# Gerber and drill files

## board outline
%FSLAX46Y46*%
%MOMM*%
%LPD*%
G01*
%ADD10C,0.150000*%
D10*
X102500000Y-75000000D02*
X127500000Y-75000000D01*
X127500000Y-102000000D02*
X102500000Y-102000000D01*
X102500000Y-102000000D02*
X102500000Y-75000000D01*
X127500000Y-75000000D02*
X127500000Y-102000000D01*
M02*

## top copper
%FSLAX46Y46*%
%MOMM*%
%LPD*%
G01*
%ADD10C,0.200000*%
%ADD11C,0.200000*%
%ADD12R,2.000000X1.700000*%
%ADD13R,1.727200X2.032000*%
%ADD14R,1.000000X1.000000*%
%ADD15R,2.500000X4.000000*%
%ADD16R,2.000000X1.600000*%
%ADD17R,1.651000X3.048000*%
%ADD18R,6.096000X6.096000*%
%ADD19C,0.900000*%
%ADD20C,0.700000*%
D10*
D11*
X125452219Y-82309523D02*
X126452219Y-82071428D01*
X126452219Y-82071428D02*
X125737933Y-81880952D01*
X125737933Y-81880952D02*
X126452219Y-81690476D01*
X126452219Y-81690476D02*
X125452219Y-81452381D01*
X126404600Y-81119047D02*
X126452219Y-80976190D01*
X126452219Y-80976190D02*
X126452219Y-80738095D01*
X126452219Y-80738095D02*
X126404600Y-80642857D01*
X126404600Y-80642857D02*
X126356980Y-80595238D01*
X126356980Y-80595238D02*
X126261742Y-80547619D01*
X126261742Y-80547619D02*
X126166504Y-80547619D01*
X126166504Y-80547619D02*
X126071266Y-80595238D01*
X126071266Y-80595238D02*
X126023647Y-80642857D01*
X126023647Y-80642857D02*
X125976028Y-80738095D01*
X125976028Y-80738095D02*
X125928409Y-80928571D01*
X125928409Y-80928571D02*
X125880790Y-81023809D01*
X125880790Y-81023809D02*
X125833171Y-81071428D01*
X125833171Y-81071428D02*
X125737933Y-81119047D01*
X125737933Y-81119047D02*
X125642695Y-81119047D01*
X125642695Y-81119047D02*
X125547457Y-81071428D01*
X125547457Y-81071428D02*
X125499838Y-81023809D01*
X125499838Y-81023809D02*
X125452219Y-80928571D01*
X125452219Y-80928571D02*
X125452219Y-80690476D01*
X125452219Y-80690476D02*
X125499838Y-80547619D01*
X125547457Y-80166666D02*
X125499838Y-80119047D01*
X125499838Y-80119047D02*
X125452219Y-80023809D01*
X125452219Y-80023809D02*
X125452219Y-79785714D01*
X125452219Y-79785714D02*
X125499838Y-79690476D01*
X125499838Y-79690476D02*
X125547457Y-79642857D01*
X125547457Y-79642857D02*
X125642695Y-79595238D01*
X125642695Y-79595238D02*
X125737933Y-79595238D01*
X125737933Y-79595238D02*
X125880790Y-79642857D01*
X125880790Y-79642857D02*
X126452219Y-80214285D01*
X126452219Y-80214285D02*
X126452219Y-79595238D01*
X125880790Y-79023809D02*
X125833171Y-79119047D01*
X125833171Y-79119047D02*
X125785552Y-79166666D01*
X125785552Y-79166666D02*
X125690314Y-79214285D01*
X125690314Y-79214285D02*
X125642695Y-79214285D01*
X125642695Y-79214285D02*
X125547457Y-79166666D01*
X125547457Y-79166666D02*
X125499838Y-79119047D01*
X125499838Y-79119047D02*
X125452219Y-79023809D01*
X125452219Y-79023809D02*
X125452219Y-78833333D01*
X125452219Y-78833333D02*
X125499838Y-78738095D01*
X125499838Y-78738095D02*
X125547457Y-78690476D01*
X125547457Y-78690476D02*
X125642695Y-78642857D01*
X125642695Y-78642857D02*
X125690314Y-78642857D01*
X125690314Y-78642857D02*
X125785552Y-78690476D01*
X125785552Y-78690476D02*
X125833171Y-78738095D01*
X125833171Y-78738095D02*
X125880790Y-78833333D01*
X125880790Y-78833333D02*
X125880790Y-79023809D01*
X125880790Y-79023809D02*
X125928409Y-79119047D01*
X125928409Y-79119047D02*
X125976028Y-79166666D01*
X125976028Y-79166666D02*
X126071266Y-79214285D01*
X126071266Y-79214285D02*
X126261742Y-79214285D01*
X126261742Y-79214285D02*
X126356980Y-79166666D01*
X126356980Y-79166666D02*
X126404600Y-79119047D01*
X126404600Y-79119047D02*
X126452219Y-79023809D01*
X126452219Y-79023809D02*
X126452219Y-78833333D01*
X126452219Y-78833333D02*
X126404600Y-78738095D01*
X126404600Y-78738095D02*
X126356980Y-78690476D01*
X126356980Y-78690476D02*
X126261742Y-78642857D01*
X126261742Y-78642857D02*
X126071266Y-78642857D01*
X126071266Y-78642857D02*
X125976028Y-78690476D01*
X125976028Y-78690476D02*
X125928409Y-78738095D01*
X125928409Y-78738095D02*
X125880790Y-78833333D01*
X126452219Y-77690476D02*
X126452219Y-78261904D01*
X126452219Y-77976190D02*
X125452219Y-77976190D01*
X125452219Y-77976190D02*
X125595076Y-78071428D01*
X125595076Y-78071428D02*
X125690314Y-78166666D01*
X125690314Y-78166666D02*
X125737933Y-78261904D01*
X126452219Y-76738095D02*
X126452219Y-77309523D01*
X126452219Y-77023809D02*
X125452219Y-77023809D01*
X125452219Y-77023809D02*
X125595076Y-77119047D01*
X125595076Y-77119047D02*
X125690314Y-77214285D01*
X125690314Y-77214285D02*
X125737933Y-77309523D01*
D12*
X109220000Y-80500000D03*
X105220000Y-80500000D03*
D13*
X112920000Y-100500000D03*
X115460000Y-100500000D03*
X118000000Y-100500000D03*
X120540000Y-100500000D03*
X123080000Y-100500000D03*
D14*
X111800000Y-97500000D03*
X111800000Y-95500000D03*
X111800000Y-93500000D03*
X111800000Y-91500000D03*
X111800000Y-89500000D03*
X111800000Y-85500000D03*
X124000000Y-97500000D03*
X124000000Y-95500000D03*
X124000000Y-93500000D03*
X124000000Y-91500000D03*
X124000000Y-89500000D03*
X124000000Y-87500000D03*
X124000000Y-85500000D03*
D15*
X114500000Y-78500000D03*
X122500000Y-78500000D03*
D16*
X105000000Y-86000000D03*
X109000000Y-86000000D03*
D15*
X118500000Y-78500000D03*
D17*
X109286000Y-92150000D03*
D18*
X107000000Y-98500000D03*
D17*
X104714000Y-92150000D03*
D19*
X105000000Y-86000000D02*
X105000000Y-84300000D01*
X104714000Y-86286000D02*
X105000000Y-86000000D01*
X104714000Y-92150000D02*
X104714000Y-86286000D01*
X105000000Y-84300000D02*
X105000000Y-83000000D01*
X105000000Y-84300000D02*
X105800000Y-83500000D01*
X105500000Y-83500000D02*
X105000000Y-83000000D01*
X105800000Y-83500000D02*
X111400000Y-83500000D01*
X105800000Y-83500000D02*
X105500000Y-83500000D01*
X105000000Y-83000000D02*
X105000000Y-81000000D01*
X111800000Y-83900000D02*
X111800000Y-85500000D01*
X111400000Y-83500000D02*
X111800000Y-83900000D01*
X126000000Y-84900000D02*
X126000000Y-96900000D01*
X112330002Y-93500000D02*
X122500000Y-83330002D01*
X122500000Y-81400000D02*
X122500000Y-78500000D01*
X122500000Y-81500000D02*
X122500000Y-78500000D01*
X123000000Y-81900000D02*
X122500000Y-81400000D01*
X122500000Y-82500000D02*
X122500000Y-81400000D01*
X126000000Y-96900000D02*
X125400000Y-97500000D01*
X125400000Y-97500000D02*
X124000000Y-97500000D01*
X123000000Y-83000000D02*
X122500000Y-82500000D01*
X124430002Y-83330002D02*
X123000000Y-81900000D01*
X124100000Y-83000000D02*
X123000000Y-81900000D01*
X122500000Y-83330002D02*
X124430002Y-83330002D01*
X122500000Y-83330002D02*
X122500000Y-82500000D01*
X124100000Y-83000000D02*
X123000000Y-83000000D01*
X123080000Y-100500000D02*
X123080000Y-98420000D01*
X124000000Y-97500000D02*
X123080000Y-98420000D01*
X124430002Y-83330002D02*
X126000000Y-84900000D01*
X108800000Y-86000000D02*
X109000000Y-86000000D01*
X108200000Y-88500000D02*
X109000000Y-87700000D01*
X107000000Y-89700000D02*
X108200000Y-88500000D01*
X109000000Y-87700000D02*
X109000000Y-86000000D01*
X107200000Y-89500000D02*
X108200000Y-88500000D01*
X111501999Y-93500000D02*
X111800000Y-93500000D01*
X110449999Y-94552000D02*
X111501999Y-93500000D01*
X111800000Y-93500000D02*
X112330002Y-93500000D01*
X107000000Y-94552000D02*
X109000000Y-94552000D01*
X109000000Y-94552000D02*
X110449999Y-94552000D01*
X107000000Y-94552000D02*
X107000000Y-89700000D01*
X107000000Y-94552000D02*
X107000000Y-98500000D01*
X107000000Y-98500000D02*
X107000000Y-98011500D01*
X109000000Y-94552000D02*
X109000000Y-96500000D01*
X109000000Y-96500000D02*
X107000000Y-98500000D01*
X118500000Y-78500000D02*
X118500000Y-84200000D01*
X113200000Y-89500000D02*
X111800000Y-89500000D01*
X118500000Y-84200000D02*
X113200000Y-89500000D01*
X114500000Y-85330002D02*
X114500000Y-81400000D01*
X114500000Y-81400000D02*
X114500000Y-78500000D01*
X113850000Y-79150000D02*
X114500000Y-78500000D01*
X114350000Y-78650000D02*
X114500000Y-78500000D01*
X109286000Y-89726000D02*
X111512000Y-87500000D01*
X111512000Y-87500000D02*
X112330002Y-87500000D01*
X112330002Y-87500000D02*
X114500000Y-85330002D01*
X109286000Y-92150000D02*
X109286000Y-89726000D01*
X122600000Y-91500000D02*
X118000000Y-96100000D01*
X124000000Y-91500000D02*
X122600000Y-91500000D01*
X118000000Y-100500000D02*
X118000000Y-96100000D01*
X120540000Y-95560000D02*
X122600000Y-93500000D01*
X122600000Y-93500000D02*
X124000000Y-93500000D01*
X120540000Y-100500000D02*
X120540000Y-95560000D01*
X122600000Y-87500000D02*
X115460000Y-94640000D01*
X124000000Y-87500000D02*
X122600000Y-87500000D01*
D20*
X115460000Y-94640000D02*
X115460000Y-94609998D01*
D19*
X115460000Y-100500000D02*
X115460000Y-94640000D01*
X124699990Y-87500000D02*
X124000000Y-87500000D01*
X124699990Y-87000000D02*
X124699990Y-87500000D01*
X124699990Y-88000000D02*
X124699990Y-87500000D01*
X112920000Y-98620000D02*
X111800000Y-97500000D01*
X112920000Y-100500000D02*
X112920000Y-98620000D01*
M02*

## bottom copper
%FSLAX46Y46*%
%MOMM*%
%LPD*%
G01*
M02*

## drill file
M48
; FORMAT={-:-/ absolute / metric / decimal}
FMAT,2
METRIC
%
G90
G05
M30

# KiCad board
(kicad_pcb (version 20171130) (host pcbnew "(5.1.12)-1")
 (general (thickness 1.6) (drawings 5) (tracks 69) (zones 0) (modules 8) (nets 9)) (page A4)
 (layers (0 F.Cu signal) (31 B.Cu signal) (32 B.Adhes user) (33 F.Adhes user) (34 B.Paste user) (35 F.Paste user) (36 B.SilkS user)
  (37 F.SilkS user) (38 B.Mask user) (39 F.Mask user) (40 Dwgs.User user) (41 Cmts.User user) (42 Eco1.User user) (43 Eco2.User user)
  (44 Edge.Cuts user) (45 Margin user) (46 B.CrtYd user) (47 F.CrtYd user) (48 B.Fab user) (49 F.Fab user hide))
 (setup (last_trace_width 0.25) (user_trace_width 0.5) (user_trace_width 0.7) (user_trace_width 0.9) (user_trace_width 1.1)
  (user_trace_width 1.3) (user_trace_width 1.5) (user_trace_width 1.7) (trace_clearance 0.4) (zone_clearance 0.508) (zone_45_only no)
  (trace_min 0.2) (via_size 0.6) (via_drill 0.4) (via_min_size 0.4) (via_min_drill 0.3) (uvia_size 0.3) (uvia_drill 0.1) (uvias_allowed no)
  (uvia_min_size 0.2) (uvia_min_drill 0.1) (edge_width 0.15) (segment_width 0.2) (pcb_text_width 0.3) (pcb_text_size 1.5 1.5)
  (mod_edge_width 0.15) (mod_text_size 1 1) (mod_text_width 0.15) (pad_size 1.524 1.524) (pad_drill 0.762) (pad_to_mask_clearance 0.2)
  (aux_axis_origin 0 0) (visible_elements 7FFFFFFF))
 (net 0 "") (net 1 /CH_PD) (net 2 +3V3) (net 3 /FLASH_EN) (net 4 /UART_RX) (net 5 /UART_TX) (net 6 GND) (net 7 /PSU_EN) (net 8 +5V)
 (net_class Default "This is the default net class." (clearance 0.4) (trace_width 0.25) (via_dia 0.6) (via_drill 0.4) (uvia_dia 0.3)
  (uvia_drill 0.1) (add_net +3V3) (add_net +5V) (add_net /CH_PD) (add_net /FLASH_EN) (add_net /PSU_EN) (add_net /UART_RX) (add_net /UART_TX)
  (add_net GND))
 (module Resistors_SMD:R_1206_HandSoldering (layer F.Cu) (at 107.22 80.5 180)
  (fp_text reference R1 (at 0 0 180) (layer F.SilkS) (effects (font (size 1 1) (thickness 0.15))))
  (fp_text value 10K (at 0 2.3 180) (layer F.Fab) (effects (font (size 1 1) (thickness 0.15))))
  (pad 1 smd rect (at -2 0 180) (size 2 1.7) (layers F.Cu F.Paste F.Mask) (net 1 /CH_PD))
  (pad 2 smd rect (at 2 0 180) (size 2 1.7) (layers F.Cu F.Paste F.Mask) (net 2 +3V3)))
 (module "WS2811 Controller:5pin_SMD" (layer F.Cu) (at 112.92 100.5)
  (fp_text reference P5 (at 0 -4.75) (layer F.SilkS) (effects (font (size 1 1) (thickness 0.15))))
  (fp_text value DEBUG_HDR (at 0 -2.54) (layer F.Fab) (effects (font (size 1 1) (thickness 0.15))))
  (pad 1 smd rect (at 0 0) (size 1.7272 2.032) (layers F.Cu F.Paste F.Mask) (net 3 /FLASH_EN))
  (pad 2 smd rect (at 2.54 0) (size 1.7272 2.032) (layers F.Cu F.Paste F.Mask) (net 1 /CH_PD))
  (pad 3 smd rect (at 5.08 0) (size 1.7272 2.032) (layers F.Cu F.Paste F.Mask) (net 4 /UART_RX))
  (pad 4 smd rect (at 7.62 0) (size 1.7272 2.032) (layers F.Cu F.Paste F.Mask) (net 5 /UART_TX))
  (pad 5 smd rect (at 10.16 0) (size 1.7272 2.032) (layers F.Cu F.Paste F.Mask) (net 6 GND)))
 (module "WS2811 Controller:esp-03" (layer F.Cu) (at 117.9 91.6)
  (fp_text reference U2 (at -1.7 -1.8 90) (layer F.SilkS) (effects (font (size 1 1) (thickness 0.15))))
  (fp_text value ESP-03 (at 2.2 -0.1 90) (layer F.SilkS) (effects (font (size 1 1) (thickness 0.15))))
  (pad 14 smd rect (at -6.1 5.9) (size 1 1) (layers F.Cu F.Paste F.Mask) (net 3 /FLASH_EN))
  (pad 13 smd rect (at -6.1 3.9) (size 1 1) (layers F.Cu F.Paste F.Mask))
  (pad 12 smd rect (at -6.1 1.9) (size 1 1) (layers F.Cu F.Paste F.Mask) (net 6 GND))
  (pad 11 smd rect (at -6.1 -0.1) (size 1 1) (layers F.Cu F.Paste F.Mask))
  (pad 10 smd rect (at -6.1 -2.1) (size 1 1) (layers F.Cu F.Paste F.Mask) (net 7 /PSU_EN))
  (pad 8 smd rect (at -6.1 -6.1) (size 1 1) (layers F.Cu F.Paste F.Mask) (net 2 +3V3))
  (pad 1 smd rect (at 6.1 5.9) (size 1 1) (layers F.Cu F.Paste F.Mask) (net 6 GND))
  (pad 2 smd rect (at 6.1 3.9) (size 1 1) (layers F.Cu F.Paste F.Mask))
  (pad 3 smd rect (at 6.1 1.9) (size 1 1) (layers F.Cu F.Paste F.Mask) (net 5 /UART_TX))
  (pad 4 smd rect (at 6.1 -0.1) (size 1 1) (layers F.Cu F.Paste F.Mask) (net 4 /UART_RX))
  (pad 5 smd rect (at 6.1 -2.1) (size 1 1) (layers F.Cu F.Paste F.Mask))
  (pad 6 smd rect (at 6.1 -4.1) (size 1 1) (layers F.Cu F.Paste F.Mask) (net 1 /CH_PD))
  (pad 7 smd rect (at 6.1 -6.1) (size 1 1) (layers F.Cu F.Paste F.Mask)))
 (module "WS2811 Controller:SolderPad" (layer F.Cu) (at 114.5 78.5 270)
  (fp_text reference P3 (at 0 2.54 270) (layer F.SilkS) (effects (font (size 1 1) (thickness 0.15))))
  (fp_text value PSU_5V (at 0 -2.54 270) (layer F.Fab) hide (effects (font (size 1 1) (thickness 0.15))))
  (pad 1 smd rect (at 0 0 270) (size 4 2.5) (layers F.Cu F.Paste F.Mask) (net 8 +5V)))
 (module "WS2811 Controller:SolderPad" (layer F.Cu) (at 122.5 78.5 270)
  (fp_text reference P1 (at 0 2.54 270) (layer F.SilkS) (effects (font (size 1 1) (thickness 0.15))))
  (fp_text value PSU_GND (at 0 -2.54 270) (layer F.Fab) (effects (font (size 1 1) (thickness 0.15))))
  (pad 1 smd rect (at 0 0 270) (size 4 2.5) (layers F.Cu F.Paste F.Mask) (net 6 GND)))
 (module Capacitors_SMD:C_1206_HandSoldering (layer F.Cu) (at 107 86)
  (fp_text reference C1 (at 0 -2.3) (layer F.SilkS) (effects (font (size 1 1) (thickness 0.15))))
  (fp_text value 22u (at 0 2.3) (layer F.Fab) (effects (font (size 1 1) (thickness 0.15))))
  (pad 1 smd rect (at -2 0) (size 2 1.6) (layers F.Cu F.Paste F.Mask) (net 2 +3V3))
  (pad 2 smd rect (at 2 0) (size 2 1.6) (layers F.Cu F.Paste F.Mask) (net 6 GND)))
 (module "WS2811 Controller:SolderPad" (layer F.Cu) (at 118.5 78.5 90)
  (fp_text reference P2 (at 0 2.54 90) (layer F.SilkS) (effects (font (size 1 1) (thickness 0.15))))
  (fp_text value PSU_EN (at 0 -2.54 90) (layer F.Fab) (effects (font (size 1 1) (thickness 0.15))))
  (pad 1 smd rect (at 0 0 90) (size 4 2.5) (layers F.Cu F.Paste F.Mask) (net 7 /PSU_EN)))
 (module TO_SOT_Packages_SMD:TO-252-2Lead (layer F.Cu) (at 107 92.15 180)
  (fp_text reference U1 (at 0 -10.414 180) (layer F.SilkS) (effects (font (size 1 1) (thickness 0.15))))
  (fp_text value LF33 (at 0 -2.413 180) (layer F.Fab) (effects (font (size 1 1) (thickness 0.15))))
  (pad 1 smd rect (at -2.286 0 180) (size 1.651 3.048) (layers F.Cu F.Paste F.Mask) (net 8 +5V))
  (pad 2 smd rect (at 0 -6.35 180) (size 6.096 6.096) (layers F.Cu F.Paste F.Mask) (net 6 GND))
  (pad 3 smd rect (at 2.286 0 180) (size 1.651 3.048) (layers F.Cu F.Paste F.Mask) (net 2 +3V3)))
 (gr_line (start 102.5 75) (end 127.5 75) (layer Edge.Cuts) (width 0.15))
 (gr_line (start 127.5 102) (end 102.5 102) (layer Edge.Cuts) (width 0.15))
 (gr_line (start 102.5 102) (end 102.5 75) (layer Edge.Cuts) (width 0.15))
 (gr_line (start 127.5 75) (end 127.5 102) (layer Edge.Cuts) (width 0.15))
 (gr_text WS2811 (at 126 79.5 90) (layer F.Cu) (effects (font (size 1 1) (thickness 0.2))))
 (segment (start 105 86) (end 105 84.3) (width 0.9) (layer F.Cu) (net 2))
 (segment (start 104.714 86.286) (end 105 86) (width 0.9) (layer F.Cu) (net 2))
 (segment (start 104.714 92.15) (end 104.714 86.286) (width 0.9) (layer F.Cu) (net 2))
 (segment (start 105 84.3) (end 105 83) (width 0.9) (layer F.Cu) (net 2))
 (segment (start 105 84.3) (end 105.8 83.5) (width 0.9) (layer F.Cu) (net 2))
 (segment (start 105.5 83.5) (end 105 83) (width 0.9) (layer F.Cu) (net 2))
 (segment (start 105.8 83.5) (end 111.4 83.5) (width 0.9) (layer F.Cu) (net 2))
 (segment (start 105.8 83.5) (end 105.5 83.5) (width 0.9) (layer F.Cu) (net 2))
 (segment (start 105 83) (end 105 81) (width 0.9) (layer F.Cu) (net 2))
 (segment (start 111.8 83.9) (end 111.8 85.5) (width 0.9) (layer F.Cu) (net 2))
 (segment (start 111.4 83.5) (end 111.8 83.9) (width 0.9) (layer F.Cu) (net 2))
 (segment (start 126 84.9) (end 126 96.9) (width 0.9) (layer F.Cu) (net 6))
 (segment (start 112.330002 93.5) (end 122.5 83.330002) (width 0.9) (layer F.Cu) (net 6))
 (segment (start 122.5 81.4) (end 122.5 78.5) (width 0.9) (layer F.Cu) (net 6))
 (segment (start 122.5 81.5) (end 122.5 78.5) (width 0.9) (layer F.Cu) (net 6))
 (segment (start 123 81.9) (end 122.5 81.4) (width 0.9) (layer F.Cu) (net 6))
 (segment (start 122.5 82.5) (end 122.5 81.4) (width 0.9) (layer F.Cu) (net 6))
 (segment (start 126 96.9) (end 125.4 97.5) (width 0.9) (layer F.Cu) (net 6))
 (segment (start 125.4 97.5) (end 124 97.5) (width 0.9) (layer F.Cu) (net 6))
 (segment (start 123 83) (end 122.5 82.5) (width 0.9) (layer F.Cu) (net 6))
 (segment (start 124.430002 83.330002) (end 123 81.9) (width 0.9) (layer F.Cu) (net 6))
 (segment (start 124.1 83) (end 123 81.9) (width 0.9) (layer F.Cu) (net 6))
 (segment (start 122.5 83.330002) (end 124.430002 83.330002) (width 0.9) (layer F.Cu) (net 6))
 (segment (start 122.5 83.330002) (end 122.5 82.5) (width 0.9) (layer F.Cu) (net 6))
 (segment (start 124.1 83) (end 123 83) (width 0.9) (layer F.Cu) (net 6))
 (segment (start 123.08 100.5) (end 123.08 98.42) (width 0.9) (layer F.Cu) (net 6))
 (segment (start 124 97.5) (end 123.08 98.42) (width 0.9) (layer F.Cu) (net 6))
 (segment (start 124.430002 83.330002) (end 126 84.9) (width 0.9) (layer F.Cu) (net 6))
 (segment (start 108.8 86) (end 109 86) (width 0.9) (layer F.Cu) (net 6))
 (segment (start 108.2 88.5) (end 109 87.7) (width 0.9) (layer F.Cu) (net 6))
 (segment (start 107 89.7) (end 108.2 88.5) (width 0.9) (layer F.Cu) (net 6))
 (segment (start 109 87.7) (end 109 86) (width 0.9) (layer F.Cu) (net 6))
 (segment (start 107.2 89.5) (end 108.2 88.5) (width 0.9) (layer F.Cu) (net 6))
 (segment (start 111.501999 93.5) (end 111.8 93.5) (width 0.9) (layer F.Cu) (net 6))
 (segment (start 110.449999 94.552) (end 111.501999 93.5) (width 0.9) (layer F.Cu) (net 6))
 (segment (start 111.8 93.5) (end 112.330002 93.5) (width 0.9) (layer F.Cu) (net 6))
 (segment (start 107 94.552) (end 109 94.552) (width 0.9) (layer F.Cu) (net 6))
 (segment (start 109 94.552) (end 110.449999 94.552) (width 0.9) (layer F.Cu) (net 6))
 (segment (start 107 94.552) (end 107 89.7) (width 0.9) (layer F.Cu) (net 6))
 (segment (start 107 94.552) (end 107 98.5) (width 0.9) (layer F.Cu) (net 6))
 (segment (start 107 98.5) (end 107 98.0115) (width 0.9) (layer F.Cu) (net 6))
 (segment (start 109 94.552) (end 109 96.5) (width 0.9) (layer F.Cu) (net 6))
 (segment (start 109 96.5) (end 107 98.5) (width 0.9) (layer F.Cu) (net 6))
 (segment (start 118.5 78.5) (end 118.5 84.2) (width 0.9) (layer F.Cu) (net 7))
 (segment (start 113.2 89.5) (end 111.8 89.5) (width 0.9) (layer F.Cu) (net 7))
 (segment (start 118.5 84.2) (end 113.2 89.5) (width 0.9) (layer F.Cu) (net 7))
 (segment (start 114.5 85.330002) (end 114.5 81.4) (width 0.9) (layer F.Cu) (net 8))
 (segment (start 114.5 81.4) (end 114.5 78.5) (width 0.9) (layer F.Cu) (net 8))
 (segment (start 113.85 79.15) (end 114.5 78.5) (width 0.9) (layer F.Cu) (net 8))
 (segment (start 114.35 78.65) (end 114.5 78.5) (width 0.9) (layer F.Cu) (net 8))
 (segment (start 109.286 89.726) (end 111.512 87.5) (width 0.9) (layer F.Cu) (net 8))
 (segment (start 111.512 87.5) (end 112.330002 87.5) (width 0.9) (layer F.Cu) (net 8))
 (segment (start 112.330002 87.5) (end 114.5 85.330002) (width 0.9) (layer F.Cu) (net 8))
 (segment (start 109.286 92.15) (end 109.286 89.726) (width 0.9) (layer F.Cu) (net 8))
 (segment (start 122.6 91.5) (end 118 96.1) (width 0.9) (layer F.Cu) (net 4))
 (segment (start 124 91.5) (end 122.6 91.5) (width 0.9) (layer F.Cu) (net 4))
 (segment (start 118 100.5) (end 118 96.1) (width 0.9) (layer F.Cu) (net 4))
 (segment (start 120.54 95.56) (end 122.6 93.5) (width 0.9) (layer F.Cu) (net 5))
 (segment (start 122.6 93.5) (end 124 93.5) (width 0.9) (layer F.Cu) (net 5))
 (segment (start 120.54 100.5) (end 120.54 95.56) (width 0.9) (layer F.Cu) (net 5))
 (segment (start 122.6 87.5) (end 115.46 94.64) (width 0.9) (layer F.Cu) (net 1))
 (segment (start 124 87.5) (end 122.6 87.5) (width 0.9) (layer F.Cu) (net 1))
 (segment (start 115.46 94.64) (end 115.46 94.609998) (width 0.7) (layer F.Cu) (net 1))
 (segment (start 115.46 100.5) (end 115.46 94.64) (width 0.9) (layer F.Cu) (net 1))
 (segment (start 124.69999 87.5) (end 124 87.5) (width 0.9) (layer F.Cu) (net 1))
 (segment (start 124.69999 87) (end 124.69999 87.5) (width 0.9) (layer F.Cu) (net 1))
 (segment (start 124.69999 88) (end 124.69999 87.5) (width 0.9) (layer F.Cu) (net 1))
 (segment (start 112.92 98.62) (end 111.8 97.5) (width 0.9) (layer F.Cu) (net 3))
 (segment (start 112.92 100.5) (end 112.92 98.62) (width 0.9) (layer F.Cu) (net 3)))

